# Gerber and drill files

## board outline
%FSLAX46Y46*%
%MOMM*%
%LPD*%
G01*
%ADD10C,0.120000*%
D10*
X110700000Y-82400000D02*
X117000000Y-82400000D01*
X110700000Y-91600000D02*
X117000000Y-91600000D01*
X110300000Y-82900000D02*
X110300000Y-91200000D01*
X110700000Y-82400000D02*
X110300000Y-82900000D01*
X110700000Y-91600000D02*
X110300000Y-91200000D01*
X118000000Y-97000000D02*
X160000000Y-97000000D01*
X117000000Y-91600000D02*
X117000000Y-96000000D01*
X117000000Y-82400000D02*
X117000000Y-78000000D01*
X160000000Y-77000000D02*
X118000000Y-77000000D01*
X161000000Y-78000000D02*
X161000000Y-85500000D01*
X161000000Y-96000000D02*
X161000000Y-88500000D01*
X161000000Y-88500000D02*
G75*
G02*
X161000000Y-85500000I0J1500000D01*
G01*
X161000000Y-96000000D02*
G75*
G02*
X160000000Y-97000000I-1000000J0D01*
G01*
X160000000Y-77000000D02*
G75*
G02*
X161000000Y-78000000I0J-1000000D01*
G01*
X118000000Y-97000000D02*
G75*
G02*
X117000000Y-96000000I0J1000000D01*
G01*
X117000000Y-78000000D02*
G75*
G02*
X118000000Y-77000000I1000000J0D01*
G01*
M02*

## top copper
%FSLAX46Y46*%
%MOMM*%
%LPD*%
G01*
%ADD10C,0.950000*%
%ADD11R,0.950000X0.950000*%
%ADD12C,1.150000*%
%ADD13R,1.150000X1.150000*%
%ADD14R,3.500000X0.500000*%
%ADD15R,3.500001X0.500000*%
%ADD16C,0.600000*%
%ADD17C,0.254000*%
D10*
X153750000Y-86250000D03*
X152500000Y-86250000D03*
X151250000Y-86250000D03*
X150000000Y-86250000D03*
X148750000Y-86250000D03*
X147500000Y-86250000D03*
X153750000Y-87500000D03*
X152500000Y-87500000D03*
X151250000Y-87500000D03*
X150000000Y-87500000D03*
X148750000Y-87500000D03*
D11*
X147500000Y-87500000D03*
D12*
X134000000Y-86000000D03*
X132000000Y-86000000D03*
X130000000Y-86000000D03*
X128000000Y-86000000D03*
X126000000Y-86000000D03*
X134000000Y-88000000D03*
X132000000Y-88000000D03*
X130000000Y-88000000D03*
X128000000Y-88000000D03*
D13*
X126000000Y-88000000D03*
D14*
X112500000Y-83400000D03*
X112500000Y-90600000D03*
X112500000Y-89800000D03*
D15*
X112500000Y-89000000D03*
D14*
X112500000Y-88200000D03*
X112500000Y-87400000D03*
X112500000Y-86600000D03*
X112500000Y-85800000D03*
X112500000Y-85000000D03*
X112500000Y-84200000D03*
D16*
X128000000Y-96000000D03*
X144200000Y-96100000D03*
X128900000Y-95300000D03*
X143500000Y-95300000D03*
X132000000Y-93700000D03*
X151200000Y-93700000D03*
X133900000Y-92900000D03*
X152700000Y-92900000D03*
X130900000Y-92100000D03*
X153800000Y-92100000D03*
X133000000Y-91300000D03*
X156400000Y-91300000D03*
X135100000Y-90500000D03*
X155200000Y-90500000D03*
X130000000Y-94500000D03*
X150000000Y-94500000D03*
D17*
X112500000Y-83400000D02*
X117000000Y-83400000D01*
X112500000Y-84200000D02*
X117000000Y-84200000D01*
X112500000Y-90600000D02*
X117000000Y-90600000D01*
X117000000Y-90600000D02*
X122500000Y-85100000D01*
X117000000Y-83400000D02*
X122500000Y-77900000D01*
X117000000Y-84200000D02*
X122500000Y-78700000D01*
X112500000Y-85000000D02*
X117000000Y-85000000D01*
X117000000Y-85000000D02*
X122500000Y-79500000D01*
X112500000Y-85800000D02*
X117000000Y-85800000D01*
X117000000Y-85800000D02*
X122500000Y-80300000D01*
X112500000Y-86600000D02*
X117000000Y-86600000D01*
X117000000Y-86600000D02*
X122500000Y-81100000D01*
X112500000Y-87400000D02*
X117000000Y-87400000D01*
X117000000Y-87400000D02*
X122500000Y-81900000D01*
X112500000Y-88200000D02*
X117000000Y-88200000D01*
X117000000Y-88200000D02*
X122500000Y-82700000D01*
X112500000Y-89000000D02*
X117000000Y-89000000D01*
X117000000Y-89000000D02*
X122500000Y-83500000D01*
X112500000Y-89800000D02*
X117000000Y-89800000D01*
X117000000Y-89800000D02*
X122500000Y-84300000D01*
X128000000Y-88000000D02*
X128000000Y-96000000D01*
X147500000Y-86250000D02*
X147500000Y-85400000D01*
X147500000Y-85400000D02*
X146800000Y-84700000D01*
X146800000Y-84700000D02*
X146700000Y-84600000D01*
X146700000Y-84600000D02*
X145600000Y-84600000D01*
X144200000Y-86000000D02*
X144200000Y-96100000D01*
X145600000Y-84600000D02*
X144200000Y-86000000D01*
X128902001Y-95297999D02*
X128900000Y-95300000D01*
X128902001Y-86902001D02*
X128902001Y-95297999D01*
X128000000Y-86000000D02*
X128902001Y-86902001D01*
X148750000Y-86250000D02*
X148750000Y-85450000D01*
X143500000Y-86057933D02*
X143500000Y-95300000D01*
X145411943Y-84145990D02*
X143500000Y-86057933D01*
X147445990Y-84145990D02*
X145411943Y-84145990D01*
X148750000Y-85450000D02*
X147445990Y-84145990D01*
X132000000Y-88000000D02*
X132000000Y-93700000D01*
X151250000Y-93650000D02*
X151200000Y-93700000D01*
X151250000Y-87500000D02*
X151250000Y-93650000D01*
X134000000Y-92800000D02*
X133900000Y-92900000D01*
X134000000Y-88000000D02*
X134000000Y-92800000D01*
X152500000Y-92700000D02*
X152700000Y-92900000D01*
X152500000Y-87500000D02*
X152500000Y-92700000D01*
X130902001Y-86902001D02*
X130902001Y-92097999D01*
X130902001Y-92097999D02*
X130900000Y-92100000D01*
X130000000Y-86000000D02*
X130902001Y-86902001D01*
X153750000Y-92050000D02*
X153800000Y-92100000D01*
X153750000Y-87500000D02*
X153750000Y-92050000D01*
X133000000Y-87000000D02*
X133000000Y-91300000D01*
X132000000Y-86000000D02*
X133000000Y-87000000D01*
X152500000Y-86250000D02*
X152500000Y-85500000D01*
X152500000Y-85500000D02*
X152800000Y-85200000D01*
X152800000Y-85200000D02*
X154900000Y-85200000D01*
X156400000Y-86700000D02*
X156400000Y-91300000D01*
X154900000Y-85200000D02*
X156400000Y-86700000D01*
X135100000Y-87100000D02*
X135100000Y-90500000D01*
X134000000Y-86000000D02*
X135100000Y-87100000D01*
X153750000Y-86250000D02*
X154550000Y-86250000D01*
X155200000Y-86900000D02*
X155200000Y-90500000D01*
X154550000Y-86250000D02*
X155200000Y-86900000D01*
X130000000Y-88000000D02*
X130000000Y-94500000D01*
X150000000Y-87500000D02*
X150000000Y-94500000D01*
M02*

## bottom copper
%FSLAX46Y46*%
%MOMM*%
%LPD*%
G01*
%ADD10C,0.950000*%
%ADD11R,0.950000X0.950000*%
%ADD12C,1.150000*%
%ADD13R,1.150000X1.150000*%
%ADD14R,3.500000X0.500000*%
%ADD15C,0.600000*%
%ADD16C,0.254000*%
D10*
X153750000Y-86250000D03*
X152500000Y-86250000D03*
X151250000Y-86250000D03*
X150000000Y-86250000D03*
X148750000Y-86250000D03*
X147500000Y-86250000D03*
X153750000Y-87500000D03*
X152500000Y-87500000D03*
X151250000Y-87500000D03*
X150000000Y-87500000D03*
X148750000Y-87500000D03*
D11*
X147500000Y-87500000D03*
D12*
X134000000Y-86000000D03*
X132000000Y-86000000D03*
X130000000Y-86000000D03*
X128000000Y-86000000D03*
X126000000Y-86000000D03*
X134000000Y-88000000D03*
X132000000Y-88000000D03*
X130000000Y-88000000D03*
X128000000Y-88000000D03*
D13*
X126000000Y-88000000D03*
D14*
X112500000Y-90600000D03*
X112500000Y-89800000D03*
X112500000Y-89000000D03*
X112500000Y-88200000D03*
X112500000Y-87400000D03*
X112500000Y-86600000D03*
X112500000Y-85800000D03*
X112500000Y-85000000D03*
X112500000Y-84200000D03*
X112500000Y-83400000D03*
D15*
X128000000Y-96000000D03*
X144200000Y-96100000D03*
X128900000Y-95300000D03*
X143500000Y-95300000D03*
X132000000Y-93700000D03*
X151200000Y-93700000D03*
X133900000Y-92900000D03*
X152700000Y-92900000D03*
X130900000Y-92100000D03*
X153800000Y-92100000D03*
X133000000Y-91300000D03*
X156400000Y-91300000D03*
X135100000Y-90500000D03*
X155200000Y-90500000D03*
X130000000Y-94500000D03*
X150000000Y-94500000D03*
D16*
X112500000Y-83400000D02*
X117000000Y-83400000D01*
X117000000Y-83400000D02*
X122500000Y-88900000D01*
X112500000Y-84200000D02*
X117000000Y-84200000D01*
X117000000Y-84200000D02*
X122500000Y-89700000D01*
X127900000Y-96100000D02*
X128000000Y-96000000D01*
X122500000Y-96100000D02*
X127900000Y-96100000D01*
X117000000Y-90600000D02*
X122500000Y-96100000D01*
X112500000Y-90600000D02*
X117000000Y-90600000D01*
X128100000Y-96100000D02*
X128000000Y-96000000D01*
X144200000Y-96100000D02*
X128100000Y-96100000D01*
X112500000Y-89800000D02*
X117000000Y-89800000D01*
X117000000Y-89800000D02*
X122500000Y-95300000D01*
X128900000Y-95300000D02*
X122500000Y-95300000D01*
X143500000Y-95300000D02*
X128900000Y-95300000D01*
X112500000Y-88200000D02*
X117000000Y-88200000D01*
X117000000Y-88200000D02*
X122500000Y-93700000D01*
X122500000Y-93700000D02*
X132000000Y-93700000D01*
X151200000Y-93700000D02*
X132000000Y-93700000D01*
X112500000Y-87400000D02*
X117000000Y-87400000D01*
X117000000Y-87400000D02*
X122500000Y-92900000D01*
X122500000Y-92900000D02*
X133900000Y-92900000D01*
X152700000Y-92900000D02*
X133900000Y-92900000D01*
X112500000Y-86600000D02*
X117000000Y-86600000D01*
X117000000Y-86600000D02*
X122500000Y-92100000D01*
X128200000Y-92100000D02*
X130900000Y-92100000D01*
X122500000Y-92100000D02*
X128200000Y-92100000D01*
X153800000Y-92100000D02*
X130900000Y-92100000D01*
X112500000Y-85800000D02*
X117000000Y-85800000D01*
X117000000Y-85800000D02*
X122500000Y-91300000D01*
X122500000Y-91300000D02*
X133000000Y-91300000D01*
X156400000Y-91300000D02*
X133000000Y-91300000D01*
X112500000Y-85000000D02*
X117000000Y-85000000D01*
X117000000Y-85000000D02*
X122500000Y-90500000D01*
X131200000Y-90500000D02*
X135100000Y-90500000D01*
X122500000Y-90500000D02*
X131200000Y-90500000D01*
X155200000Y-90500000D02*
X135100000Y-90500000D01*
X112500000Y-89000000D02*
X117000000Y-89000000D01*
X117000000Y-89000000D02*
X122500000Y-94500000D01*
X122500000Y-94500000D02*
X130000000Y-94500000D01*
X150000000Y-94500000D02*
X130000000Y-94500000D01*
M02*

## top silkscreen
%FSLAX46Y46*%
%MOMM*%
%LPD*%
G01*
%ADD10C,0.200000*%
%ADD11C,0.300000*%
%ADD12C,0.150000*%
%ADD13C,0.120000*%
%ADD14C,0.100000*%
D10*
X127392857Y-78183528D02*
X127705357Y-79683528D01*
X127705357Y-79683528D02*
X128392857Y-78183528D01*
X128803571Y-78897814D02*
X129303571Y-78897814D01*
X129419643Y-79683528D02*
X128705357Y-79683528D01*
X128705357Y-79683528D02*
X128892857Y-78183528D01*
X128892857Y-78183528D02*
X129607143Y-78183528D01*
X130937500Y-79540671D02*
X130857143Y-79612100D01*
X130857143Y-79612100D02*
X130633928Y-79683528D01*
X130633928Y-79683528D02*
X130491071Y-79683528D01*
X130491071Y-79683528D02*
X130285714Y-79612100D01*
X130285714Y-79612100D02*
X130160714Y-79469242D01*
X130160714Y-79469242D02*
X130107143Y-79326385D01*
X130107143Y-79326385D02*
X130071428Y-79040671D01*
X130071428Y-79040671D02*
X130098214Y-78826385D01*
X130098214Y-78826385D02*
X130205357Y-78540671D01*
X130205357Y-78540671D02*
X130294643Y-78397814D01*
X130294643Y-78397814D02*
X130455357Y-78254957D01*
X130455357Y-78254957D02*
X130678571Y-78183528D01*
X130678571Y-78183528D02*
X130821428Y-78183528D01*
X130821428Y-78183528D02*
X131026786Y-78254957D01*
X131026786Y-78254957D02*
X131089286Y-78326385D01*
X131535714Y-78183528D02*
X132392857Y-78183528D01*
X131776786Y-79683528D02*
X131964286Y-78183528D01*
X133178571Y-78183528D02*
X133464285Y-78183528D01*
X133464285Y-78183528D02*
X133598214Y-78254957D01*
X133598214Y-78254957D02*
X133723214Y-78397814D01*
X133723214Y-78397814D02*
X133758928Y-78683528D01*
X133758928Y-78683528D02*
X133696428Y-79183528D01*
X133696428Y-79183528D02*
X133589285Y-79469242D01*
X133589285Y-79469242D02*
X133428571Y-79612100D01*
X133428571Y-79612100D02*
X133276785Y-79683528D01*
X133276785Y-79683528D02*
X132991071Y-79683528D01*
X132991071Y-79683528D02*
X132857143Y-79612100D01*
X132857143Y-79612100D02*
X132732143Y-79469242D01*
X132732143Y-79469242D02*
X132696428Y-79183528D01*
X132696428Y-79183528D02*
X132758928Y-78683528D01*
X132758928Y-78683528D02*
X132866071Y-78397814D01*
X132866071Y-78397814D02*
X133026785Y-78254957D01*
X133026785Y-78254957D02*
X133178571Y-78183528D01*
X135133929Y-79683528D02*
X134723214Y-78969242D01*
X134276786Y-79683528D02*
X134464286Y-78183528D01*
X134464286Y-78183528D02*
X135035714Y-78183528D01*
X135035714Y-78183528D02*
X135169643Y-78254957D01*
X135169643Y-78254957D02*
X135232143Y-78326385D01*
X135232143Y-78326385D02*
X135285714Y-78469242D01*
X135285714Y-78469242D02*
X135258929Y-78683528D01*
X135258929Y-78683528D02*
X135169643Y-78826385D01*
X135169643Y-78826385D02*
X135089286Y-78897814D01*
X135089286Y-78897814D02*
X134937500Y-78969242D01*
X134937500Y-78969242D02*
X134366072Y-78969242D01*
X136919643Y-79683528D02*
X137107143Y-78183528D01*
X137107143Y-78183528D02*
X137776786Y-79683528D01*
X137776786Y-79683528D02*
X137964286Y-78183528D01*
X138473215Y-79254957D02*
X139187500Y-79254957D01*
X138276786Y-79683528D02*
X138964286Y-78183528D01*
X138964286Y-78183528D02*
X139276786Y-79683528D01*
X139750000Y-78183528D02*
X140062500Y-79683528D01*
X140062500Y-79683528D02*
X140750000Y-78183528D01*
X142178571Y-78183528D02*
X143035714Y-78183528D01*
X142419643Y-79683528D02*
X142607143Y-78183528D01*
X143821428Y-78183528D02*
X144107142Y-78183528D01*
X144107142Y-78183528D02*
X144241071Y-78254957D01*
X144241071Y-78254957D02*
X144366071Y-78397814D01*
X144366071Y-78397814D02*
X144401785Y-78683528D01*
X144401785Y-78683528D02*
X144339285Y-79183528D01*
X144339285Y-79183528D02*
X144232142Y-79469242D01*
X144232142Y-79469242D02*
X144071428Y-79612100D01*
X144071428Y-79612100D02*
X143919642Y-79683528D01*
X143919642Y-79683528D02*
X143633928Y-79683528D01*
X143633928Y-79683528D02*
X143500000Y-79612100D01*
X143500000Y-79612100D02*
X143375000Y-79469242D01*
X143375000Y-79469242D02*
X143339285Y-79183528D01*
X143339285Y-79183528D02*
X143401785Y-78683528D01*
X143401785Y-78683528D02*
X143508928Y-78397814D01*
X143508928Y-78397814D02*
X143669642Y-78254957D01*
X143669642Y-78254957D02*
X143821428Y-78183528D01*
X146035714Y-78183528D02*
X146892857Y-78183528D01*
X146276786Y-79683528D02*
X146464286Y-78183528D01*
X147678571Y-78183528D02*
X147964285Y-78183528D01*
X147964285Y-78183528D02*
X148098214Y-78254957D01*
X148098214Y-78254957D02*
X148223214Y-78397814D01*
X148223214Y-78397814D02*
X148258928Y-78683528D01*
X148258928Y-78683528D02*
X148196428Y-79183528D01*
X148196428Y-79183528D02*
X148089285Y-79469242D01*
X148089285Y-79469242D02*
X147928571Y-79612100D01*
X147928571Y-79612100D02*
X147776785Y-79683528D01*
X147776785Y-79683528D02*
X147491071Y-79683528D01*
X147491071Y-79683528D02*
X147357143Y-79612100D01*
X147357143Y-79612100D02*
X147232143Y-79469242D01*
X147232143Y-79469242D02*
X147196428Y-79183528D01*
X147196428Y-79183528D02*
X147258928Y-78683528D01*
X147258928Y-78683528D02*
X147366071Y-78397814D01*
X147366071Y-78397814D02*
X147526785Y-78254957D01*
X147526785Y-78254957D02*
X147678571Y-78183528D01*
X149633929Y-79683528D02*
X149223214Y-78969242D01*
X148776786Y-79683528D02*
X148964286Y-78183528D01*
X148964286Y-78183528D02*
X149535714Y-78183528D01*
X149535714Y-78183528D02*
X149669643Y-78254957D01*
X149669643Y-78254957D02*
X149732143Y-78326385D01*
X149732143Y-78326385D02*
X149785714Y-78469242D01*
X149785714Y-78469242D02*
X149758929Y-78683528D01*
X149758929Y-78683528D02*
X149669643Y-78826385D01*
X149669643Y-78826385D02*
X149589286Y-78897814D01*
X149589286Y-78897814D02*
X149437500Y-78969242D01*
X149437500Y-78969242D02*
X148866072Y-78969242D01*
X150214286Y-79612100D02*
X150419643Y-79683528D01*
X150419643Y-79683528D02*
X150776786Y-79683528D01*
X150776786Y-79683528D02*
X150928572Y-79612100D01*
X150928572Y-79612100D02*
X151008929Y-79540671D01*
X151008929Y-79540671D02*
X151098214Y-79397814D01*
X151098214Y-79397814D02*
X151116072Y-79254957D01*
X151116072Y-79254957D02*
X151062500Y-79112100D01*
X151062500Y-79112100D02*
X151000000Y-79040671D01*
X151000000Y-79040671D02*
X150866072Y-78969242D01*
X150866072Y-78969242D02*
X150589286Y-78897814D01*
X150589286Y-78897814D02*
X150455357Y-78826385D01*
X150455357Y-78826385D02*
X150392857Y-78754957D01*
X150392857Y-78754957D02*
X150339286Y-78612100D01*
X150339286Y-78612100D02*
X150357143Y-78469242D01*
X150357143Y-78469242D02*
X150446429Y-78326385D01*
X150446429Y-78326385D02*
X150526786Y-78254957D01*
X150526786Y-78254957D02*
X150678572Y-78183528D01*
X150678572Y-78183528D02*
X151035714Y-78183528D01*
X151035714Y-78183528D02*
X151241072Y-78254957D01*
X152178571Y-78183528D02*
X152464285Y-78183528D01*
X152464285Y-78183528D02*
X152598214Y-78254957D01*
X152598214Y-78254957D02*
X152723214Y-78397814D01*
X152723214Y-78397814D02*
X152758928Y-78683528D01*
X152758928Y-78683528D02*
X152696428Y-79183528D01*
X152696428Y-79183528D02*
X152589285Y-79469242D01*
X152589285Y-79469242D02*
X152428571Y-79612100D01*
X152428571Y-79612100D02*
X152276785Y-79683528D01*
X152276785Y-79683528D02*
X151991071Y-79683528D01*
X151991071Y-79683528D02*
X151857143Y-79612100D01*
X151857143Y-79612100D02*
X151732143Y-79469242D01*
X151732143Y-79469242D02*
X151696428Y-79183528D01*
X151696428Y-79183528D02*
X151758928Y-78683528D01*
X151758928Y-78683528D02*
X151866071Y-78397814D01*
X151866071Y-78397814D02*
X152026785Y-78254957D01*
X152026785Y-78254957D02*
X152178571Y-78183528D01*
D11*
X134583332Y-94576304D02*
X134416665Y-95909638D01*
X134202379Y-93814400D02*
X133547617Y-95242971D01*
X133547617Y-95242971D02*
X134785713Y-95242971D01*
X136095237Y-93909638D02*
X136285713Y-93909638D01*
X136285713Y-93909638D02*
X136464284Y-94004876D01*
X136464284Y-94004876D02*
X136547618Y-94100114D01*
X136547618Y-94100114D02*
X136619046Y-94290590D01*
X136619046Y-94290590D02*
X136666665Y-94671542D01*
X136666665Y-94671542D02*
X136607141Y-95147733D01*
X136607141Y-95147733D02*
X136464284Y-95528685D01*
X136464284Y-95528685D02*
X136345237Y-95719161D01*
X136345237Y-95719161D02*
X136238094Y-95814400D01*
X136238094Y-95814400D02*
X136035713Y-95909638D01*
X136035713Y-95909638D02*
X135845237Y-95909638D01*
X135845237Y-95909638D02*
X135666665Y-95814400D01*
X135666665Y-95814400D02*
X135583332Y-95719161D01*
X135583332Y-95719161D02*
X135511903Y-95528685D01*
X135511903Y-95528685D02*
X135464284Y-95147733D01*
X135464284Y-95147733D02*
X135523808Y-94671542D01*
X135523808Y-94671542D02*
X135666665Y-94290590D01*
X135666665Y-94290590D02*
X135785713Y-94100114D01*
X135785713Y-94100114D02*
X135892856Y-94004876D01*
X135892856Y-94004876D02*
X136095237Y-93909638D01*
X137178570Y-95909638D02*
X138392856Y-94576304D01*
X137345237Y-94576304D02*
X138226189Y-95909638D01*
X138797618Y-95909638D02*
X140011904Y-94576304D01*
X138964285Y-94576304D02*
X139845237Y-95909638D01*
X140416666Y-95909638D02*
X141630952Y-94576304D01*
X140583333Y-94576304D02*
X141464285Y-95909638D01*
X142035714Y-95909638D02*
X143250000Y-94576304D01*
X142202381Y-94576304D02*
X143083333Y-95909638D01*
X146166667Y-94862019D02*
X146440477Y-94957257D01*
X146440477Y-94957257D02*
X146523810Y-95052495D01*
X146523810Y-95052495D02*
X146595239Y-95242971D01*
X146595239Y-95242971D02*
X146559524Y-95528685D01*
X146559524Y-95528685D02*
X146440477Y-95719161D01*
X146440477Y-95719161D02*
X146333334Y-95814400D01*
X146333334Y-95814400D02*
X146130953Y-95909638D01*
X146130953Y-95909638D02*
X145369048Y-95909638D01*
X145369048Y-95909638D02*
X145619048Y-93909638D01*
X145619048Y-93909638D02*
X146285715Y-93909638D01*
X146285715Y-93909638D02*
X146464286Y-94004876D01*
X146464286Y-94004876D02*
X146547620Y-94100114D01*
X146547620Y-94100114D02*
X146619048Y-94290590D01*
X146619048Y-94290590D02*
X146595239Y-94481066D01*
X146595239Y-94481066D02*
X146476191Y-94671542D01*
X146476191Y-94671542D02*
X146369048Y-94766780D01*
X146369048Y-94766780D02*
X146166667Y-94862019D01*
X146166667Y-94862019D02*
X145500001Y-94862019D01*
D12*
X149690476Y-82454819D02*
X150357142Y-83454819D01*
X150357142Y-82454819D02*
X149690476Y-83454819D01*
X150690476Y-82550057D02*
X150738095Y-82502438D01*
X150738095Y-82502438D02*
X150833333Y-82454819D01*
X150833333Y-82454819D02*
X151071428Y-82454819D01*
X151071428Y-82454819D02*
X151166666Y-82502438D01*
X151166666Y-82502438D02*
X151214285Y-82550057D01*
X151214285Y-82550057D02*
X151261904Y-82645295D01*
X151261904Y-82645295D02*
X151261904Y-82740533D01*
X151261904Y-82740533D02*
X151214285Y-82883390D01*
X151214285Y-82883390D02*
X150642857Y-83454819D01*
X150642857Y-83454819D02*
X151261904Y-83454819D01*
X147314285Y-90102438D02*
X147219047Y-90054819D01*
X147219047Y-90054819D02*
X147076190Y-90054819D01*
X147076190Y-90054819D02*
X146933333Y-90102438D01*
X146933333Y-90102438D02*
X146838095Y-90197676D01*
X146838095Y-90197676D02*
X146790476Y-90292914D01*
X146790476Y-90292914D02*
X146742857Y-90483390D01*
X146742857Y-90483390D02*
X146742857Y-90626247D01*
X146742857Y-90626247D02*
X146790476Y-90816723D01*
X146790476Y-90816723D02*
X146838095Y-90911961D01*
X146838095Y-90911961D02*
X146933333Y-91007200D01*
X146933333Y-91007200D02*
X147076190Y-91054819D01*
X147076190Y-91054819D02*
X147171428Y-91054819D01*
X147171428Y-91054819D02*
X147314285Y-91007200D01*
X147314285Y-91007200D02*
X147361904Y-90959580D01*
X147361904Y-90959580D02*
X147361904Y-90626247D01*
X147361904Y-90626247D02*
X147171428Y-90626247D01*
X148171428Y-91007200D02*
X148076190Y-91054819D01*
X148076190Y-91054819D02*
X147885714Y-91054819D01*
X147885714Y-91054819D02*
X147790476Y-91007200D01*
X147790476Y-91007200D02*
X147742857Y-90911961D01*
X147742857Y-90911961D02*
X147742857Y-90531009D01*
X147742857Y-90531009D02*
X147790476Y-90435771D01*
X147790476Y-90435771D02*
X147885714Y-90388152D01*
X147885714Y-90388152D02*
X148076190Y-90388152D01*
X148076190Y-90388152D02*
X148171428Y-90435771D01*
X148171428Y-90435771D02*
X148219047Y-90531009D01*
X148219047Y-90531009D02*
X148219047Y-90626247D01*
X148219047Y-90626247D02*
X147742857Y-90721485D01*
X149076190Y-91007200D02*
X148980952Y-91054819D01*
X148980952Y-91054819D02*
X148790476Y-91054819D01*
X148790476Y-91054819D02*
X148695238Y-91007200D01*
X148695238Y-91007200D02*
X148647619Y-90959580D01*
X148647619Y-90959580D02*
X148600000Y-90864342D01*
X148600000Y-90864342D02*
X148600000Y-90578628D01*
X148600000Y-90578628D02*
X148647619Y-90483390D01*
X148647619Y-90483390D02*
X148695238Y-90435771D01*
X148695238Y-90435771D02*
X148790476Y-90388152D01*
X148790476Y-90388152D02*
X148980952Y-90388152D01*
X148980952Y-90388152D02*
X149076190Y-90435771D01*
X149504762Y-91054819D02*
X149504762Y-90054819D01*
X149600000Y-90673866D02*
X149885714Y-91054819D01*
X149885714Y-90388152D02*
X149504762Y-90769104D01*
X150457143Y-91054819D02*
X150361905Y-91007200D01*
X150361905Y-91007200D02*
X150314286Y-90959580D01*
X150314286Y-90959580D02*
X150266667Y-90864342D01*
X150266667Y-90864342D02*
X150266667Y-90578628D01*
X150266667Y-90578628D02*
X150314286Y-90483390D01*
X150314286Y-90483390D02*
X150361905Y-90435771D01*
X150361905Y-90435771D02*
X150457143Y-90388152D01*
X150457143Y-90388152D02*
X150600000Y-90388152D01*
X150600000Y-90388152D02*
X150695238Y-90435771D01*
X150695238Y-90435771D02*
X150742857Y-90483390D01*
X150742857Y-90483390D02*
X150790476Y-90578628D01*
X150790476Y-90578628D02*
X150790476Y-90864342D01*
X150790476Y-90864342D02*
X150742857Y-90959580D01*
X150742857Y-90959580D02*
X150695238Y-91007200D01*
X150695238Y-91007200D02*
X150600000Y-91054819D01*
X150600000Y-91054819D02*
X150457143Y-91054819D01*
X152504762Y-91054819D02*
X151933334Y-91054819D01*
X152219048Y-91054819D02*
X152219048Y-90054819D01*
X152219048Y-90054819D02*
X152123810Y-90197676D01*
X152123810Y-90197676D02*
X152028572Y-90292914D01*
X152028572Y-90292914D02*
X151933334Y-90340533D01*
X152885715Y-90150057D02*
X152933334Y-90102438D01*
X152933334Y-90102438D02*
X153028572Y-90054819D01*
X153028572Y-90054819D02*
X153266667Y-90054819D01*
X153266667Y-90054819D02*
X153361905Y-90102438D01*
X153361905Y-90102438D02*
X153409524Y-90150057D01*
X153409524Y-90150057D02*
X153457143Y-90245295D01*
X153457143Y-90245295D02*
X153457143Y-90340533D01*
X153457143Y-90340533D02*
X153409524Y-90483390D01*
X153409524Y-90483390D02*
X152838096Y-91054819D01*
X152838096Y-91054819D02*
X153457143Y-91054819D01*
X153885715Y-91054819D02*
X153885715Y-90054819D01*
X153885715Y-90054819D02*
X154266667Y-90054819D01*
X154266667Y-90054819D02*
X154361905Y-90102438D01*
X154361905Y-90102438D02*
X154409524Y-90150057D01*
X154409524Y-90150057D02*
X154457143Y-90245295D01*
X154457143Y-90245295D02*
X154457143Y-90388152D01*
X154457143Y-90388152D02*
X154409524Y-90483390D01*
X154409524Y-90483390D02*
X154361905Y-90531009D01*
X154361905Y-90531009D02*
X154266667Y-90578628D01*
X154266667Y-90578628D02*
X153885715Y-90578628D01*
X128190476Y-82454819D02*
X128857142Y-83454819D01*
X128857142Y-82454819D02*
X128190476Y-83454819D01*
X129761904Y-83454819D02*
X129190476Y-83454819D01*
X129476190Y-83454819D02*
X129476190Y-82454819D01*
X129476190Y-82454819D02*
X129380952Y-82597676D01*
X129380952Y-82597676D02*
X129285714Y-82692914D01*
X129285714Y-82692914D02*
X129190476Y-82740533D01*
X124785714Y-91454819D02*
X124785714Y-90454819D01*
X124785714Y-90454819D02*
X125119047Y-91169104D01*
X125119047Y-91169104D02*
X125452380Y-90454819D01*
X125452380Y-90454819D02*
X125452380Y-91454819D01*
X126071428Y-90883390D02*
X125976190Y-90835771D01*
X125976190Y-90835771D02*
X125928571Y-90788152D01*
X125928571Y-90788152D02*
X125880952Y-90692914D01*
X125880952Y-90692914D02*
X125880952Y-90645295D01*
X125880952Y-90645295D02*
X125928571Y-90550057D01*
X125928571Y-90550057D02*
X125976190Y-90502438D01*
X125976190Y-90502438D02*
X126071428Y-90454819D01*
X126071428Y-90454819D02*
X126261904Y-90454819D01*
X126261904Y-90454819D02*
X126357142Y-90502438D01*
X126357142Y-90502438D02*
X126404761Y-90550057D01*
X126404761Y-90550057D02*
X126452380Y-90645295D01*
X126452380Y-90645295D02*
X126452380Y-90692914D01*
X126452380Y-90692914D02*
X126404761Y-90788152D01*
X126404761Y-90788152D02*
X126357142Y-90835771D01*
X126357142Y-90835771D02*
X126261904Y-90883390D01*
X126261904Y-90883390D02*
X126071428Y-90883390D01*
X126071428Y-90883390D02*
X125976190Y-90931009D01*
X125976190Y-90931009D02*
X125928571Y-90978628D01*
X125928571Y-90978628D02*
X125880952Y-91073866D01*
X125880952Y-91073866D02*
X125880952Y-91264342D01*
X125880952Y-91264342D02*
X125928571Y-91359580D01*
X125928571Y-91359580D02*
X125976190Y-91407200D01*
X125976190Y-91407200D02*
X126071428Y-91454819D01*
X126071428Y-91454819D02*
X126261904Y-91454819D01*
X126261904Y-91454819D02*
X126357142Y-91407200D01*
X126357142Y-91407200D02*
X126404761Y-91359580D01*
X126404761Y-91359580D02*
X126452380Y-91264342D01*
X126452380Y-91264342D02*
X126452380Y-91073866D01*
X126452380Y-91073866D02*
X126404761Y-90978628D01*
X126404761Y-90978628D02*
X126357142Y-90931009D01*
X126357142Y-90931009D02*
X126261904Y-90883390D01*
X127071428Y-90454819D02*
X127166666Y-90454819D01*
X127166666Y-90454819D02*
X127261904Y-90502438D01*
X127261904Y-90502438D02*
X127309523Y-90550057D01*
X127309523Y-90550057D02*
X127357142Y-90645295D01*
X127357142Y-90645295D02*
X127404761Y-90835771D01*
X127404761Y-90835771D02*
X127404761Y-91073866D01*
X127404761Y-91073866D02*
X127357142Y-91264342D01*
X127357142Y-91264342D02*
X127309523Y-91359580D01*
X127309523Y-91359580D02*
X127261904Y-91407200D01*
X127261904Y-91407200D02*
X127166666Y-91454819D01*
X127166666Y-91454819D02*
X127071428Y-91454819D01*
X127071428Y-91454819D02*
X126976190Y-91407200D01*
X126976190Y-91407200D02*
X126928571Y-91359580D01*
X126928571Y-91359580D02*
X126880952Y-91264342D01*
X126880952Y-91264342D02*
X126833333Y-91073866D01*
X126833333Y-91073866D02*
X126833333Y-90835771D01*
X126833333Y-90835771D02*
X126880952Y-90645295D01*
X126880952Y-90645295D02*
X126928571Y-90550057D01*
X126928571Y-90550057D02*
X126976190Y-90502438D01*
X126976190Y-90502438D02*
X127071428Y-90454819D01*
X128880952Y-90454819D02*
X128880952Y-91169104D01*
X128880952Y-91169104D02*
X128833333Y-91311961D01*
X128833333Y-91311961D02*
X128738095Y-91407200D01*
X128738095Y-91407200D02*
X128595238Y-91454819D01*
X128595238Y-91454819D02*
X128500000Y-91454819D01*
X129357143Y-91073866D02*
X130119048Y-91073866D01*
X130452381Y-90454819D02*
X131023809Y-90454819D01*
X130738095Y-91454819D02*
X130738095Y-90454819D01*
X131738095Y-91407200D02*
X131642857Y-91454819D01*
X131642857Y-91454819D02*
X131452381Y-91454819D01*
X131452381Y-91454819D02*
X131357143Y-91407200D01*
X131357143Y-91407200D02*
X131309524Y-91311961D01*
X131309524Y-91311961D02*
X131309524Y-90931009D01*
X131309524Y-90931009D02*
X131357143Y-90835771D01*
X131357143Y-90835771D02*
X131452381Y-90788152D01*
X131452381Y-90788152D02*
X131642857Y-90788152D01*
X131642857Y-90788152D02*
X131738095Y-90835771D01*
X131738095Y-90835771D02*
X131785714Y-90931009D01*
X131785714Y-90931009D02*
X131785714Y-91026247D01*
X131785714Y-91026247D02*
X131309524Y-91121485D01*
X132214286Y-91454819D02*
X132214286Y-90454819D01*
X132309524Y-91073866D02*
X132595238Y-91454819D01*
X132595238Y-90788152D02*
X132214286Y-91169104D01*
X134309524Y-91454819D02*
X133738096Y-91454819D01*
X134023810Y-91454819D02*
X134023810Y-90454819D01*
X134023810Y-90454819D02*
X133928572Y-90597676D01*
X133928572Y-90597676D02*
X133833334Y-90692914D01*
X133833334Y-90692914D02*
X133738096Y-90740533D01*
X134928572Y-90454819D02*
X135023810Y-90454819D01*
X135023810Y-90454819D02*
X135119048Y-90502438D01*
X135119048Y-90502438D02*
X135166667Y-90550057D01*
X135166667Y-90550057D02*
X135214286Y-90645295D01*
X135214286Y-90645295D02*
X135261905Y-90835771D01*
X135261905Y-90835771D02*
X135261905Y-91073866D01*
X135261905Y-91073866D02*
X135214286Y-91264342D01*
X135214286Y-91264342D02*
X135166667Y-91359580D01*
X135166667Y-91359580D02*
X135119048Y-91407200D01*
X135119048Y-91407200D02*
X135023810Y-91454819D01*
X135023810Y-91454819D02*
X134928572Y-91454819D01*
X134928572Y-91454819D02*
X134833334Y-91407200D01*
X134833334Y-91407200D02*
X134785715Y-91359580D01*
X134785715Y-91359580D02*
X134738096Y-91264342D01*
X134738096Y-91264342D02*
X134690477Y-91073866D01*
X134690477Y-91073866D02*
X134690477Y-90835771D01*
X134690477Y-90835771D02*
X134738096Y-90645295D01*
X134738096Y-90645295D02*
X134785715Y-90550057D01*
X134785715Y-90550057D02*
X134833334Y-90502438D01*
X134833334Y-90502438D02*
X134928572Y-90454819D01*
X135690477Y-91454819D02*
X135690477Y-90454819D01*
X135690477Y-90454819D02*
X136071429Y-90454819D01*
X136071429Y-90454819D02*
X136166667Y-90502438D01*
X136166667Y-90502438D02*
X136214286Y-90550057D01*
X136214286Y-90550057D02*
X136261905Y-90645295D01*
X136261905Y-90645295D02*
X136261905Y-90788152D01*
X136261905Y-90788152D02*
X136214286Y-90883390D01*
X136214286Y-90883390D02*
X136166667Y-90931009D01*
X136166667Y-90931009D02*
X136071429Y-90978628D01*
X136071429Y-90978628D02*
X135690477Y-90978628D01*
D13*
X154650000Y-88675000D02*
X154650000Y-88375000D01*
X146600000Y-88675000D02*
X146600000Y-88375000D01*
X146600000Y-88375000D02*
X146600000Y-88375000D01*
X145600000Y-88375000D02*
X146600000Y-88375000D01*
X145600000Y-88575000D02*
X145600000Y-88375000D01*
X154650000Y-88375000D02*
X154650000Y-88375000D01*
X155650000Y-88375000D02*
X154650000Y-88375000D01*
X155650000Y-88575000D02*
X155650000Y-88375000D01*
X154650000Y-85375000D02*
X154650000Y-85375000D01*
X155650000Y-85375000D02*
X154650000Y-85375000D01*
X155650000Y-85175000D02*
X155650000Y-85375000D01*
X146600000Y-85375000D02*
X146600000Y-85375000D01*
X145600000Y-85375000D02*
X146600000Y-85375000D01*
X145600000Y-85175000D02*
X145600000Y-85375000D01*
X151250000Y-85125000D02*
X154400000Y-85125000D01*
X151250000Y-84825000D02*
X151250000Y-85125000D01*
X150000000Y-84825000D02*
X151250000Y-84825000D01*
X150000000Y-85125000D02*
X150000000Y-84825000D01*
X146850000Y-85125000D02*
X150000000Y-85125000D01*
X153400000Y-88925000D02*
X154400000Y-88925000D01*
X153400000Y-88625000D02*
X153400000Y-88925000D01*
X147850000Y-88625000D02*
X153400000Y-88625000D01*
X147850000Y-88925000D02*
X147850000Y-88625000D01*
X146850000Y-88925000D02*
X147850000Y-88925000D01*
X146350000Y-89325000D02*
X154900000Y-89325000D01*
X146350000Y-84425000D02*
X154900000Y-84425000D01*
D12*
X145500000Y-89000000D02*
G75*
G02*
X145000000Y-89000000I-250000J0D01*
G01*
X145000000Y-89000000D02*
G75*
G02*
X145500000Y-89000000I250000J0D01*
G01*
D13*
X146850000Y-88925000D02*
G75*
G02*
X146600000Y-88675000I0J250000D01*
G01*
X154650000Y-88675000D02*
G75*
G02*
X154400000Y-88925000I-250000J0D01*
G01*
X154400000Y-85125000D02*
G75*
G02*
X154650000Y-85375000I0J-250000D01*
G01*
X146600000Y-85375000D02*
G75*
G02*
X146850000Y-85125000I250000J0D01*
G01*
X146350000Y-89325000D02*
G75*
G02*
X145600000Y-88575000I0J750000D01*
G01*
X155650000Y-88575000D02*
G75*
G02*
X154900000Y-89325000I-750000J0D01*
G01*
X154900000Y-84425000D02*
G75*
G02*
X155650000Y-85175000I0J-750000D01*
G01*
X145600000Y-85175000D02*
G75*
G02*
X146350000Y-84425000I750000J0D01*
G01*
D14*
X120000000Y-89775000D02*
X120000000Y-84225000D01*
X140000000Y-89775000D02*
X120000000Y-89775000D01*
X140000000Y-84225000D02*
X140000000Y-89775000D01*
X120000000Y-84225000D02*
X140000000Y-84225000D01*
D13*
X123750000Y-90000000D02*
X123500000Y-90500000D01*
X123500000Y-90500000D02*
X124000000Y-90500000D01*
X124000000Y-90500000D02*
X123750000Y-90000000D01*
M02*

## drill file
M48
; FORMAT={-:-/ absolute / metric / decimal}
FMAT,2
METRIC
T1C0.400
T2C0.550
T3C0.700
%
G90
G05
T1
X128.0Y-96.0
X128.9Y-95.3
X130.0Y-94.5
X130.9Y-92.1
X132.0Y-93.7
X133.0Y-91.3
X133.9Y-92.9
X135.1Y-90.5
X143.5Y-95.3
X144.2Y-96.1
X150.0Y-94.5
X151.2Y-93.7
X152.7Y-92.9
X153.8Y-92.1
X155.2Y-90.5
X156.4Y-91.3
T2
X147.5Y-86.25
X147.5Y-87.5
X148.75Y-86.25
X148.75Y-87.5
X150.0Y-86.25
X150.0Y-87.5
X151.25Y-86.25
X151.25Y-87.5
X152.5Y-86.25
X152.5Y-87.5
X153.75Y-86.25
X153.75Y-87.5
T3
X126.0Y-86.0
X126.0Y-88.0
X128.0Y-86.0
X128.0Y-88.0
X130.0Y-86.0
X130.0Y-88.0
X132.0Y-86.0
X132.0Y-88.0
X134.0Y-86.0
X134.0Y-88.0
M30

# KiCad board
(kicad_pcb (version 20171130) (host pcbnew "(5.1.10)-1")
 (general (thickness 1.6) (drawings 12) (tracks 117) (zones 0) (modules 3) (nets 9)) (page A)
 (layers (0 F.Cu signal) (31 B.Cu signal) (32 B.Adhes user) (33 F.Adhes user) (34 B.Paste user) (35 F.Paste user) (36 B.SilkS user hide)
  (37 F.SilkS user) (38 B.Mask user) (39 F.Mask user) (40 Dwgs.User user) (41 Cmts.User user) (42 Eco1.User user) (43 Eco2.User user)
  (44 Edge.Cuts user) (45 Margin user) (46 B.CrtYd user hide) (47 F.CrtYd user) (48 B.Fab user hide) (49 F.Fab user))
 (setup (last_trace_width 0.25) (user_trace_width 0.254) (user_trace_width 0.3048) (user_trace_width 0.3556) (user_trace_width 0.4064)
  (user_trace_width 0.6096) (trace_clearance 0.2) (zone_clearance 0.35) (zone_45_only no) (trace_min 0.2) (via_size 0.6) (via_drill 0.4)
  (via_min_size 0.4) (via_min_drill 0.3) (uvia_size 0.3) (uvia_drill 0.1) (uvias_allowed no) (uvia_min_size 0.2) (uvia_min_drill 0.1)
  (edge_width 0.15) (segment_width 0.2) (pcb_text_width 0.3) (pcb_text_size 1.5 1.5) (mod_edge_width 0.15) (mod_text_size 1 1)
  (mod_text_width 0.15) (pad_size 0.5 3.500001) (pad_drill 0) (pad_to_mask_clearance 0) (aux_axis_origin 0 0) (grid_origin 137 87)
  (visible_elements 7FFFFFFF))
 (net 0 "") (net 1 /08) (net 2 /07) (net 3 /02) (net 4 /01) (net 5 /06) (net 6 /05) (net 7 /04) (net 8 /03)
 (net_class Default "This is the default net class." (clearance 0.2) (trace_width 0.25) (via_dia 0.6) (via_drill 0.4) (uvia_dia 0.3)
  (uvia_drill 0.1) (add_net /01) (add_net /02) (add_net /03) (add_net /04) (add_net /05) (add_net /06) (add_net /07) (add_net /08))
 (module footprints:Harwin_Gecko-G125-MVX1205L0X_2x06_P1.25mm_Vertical (layer F.Cu) (at 147.5 87.5)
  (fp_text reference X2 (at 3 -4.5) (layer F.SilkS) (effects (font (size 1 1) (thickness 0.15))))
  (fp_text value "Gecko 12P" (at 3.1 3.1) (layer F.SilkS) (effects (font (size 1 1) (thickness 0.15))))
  (fp_line (start 7.15 1.175) (end 7.15 0.875) (layer F.SilkS) (width 0.12))
  (fp_line (start -0.9 1.175) (end -0.9 0.875) (layer F.SilkS) (width 0.12))
  (fp_line (start -0.9 0.875) (end -0.9 0.875) (layer F.SilkS) (width 0.12))
  (fp_line (start -1.9 0.875) (end -0.9 0.875) (layer F.SilkS) (width 0.12))
  (fp_line (start -1.9 1.075) (end -1.9 0.875) (layer F.SilkS) (width 0.12))
  (fp_line (start 7.15 0.875) (end 7.15 0.875) (layer F.SilkS) (width 0.12))
  (fp_line (start 8.15 0.875) (end 7.15 0.875) (layer F.SilkS) (width 0.12))
  (fp_line (start 8.15 1.075) (end 8.15 0.875) (layer F.SilkS) (width 0.12))
  (fp_line (start 7.15 -2.125) (end 7.15 -2.125) (layer F.SilkS) (width 0.12))
  (fp_line (start 8.15 -2.125) (end 7.15 -2.125) (layer F.SilkS) (width 0.12))
  (fp_line (start 8.15 -2.325) (end 8.15 -2.125) (layer F.SilkS) (width 0.12))
  (fp_line (start -0.9 -2.125) (end -0.9 -2.125) (layer F.SilkS) (width 0.12))
  (fp_line (start -1.9 -2.125) (end -0.9 -2.125) (layer F.SilkS) (width 0.12))
  (fp_line (start -1.9 -2.325) (end -1.9 -2.125) (layer F.SilkS) (width 0.12))
  (fp_line (start 3.75 -2.375) (end 6.9 -2.375) (layer F.SilkS) (width 0.12))
  (fp_line (start 3.75 -2.675) (end 3.75 -2.375) (layer F.SilkS) (width 0.12))
  (fp_line (start 2.5 -2.675) (end 3.75 -2.675) (layer F.SilkS) (width 0.12))
  (fp_line (start 2.5 -2.375) (end 2.5 -2.675) (layer F.SilkS) (width 0.12))
  (fp_line (start -0.65 -2.375) (end 2.5 -2.375) (layer F.SilkS) (width 0.12))
  (fp_line (start 5.9 1.425) (end 6.9 1.425) (layer F.SilkS) (width 0.12))
  (fp_line (start 5.9 1.125) (end 5.9 1.425) (layer F.SilkS) (width 0.12))
  (fp_line (start 0.35 1.125) (end 5.9 1.125) (layer F.SilkS) (width 0.12))
  (fp_line (start 0.35 1.425) (end 0.35 1.125) (layer F.SilkS) (width 0.12))
  (fp_line (start -0.65 1.425) (end 0.35 1.425) (layer F.SilkS) (width 0.12))
  (fp_line (start -1.15 1.825) (end 7.4 1.825) (layer F.SilkS) (width 0.12))
  (fp_line (start -1.15 -3.075) (end 7.4 -3.075) (layer F.SilkS) (width 0.12))
  (fp_circle (center -2.25 1.5) (end -2 1.5) (layer F.SilkS) (width 0.15))
  (fp_arc (start -0.65 1.175) (end -0.65 1.425) (angle 90) (layer F.SilkS) (width 0.12))
  (fp_arc (start 6.9 1.175) (end 7.15 1.175) (angle 90) (layer F.SilkS) (width 0.12))
  (fp_arc (start 6.9 -2.125) (end 6.9 -2.375) (angle 90) (layer F.SilkS) (width 0.12))
  (fp_arc (start -0.65 -2.125) (end -0.9 -2.125) (angle 90) (layer F.SilkS) (width 0.12))
  (fp_arc (start -1.15 1.075) (end -1.15 1.825) (angle 90) (layer F.SilkS) (width 0.12))
  (fp_arc (start 7.4 1.075) (end 8.15 1.075) (angle 90) (layer F.SilkS) (width 0.12))
  (fp_arc (start 7.4 -2.325) (end 7.4 -3.075) (angle 90) (layer F.SilkS) (width 0.12))
  (fp_arc (start -1.15 -2.325) (end -1.9 -2.325) (angle 90) (layer F.SilkS) (width 0.12))
  (pad 12 thru_hole circle (at 6.25 -1.25) (size 0.95 0.95) (drill 0.55) (layers *.Cu *.Mask) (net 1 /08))
  (pad 11 thru_hole circle (at 5 -1.25) (size 0.95 0.95) (drill 0.55) (layers *.Cu *.Mask) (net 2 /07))
  (pad 10 thru_hole circle (at 3.75 -1.25) (size 0.95 0.95) (drill 0.55) (layers *.Cu *.Mask))
  (pad 9 thru_hole circle (at 2.5 -1.25) (size 0.95 0.95) (drill 0.55) (layers *.Cu *.Mask))
  (pad 8 thru_hole circle (at 1.25 -1.25) (size 0.95 0.95) (drill 0.55) (layers *.Cu *.Mask) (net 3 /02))
  (pad 7 thru_hole circle (at 0 -1.25) (size 0.95 0.95) (drill 0.55) (layers *.Cu *.Mask) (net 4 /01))
  (pad 6 thru_hole circle (at 6.25 0) (size 0.95 0.95) (drill 0.55) (layers *.Cu *.Mask) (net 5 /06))
  (pad 5 thru_hole circle (at 5 0) (size 0.95 0.95) (drill 0.55) (layers *.Cu *.Mask) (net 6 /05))
  (pad 4 thru_hole circle (at 3.75 0) (size 0.95 0.95) (drill 0.55) (layers *.Cu *.Mask) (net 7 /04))
  (pad 3 thru_hole circle (at 2.5 0) (size 0.95 0.95) (drill 0.55) (layers *.Cu *.Mask) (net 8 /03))
  (pad 2 thru_hole circle (at 1.25 0) (size 0.95 0.95) (drill 0.55) (layers *.Cu *.Mask))
  (pad 1 thru_hole rect (at 0 0) (size 0.95 0.95) (drill 0.55) (layers *.Cu *.Mask)))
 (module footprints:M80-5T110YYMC (layer F.Cu) (at 126 88)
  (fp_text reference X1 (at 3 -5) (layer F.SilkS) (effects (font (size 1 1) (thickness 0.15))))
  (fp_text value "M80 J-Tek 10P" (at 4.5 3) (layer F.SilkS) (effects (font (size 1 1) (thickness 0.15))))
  (fp_line (start -6 1.775) (end -6 -3.775) (layer F.SilkS) (width 0.1))
  (fp_line (start 14 1.775) (end -6 1.775) (layer F.SilkS) (width 0.1))
  (fp_line (start 14 -3.775) (end 14 1.775) (layer F.SilkS) (width 0.1))
  (fp_line (start -6 -3.775) (end 14 -3.775) (layer F.SilkS) (width 0.1))
  (fp_line (start -2.25 2) (end -2.5 2.5) (layer F.SilkS) (width 0.12))
  (fp_line (start -2.5 2.5) (end -2 2.5) (layer F.SilkS) (width 0.12))
  (fp_line (start -2 2.5) (end -2.25 2) (layer F.SilkS) (width 0.12))
  (pad 10 thru_hole circle (at 8 -2) (size 1.15 1.15) (drill 0.7) (layers *.Cu *.Mask) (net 1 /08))
  (pad 9 thru_hole circle (at 6 -2) (size 1.15 1.15) (drill 0.7) (layers *.Cu *.Mask) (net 2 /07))
  (pad 8 thru_hole circle (at 4 -2) (size 1.15 1.15) (drill 0.7) (layers *.Cu *.Mask) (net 5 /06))
  (pad 7 thru_hole circle (at 2 -2) (size 1.15 1.15) (drill 0.7) (layers *.Cu *.Mask) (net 3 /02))
  (pad 6 thru_hole circle (at 0 -2) (size 1.15 1.15) (drill 0.7) (layers *.Cu *.Mask))
  (pad 5 thru_hole circle (at 8 0) (size 1.15 1.15) (drill 0.7) (layers *.Cu *.Mask) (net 6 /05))
  (pad 4 thru_hole circle (at 6 0) (size 1.15 1.15) (drill 0.7) (layers *.Cu *.Mask) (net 7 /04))
  (pad 3 thru_hole circle (at 4 0) (size 1.15 1.15) (drill 0.7) (layers *.Cu *.Mask) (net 8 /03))
  (pad 2 thru_hole circle (at 2 0) (size 1.15 1.15) (drill 0.7) (layers *.Cu *.Mask) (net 4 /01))
  (pad 1 thru_hole rect (at 0 0) (size 1.15 1.15) (drill 0.7) (layers *.Cu *.Mask)))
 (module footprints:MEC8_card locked (layer F.Cu) (at 112.5 87 90)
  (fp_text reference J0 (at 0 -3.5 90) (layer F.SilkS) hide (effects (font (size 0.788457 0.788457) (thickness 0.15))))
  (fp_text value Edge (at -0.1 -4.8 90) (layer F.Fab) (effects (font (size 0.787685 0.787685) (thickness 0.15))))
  (fp_line (start 4.6 -1.8) (end 4.6 4.5) (layer Edge.Cuts) (width 0.12))
  (fp_line (start -4.6 -1.8) (end -4.6 4.5) (layer Edge.Cuts) (width 0.12))
  (fp_line (start 4.1 -2.2) (end -4.2 -2.2) (layer Edge.Cuts) (width 0.12))
  (fp_line (start 4.6 -1.8) (end 4.1 -2.2) (layer Edge.Cuts) (width 0.12))
  (fp_line (start -4.6 -1.8) (end -4.2 -2.2) (layer Edge.Cuts) (width 0.12))
  (fp_line (start -10 5.5) (end -10 47.5) (layer Edge.Cuts) (width 0.12))
  (fp_line (start -4.6 4.5) (end -9 4.5) (layer Edge.Cuts) (width 0.12))
  (fp_line (start 4.6 4.5) (end 9 4.5) (layer Edge.Cuts) (width 0.12))
  (fp_line (start 10 47.5) (end 10 5.5) (layer Edge.Cuts) (width 0.12))
  (fp_line (start 9 48.5) (end 1.5 48.5) (layer Edge.Cuts) (width 0.12))
  (fp_line (start -9 48.5) (end -1.5 48.5) (layer Edge.Cuts) (width 0.12))
  (fp_arc (start 0 48.5) (end 1.5 48.5) (angle -180) (layer Edge.Cuts) (width 0.12))
  (fp_arc (start -9 47.5) (end -10 47.5) (angle -90) (layer Edge.Cuts) (width 0.12))
  (fp_arc (start 9 47.5) (end 9 48.5) (angle -90) (layer Edge.Cuts) (width 0.12))
  (fp_arc (start -9 5.5) (end -9 4.5) (angle -90) (layer Edge.Cuts) (width 0.12))
  (fp_arc (start 9 5.5) (end 10 5.5) (angle -90) (layer Edge.Cuts) (width 0.12))
  (pad 20 smd rect (at 3.6 0 90) (size 0.5 3.5) (layers F.Cu F.Paste F.Mask))
  (pad 11 smd rect (at -3.6 0 90) (size 0.5 3.5) (layers F.Cu F.Paste F.Mask))
  (pad 12 smd rect (at -2.8 0 90) (size 0.5 3.5) (layers F.Cu F.Paste F.Mask))
  (pad 13 smd rect (at -2 0 90) (size 0.5 3.500001) (layers F.Cu F.Paste F.Mask))
  (pad 14 smd rect (at -1.2 0 90) (size 0.5 3.5) (layers F.Cu F.Paste F.Mask))
  (pad 15 smd rect (at -0.4 0 90) (size 0.5 3.5) (layers F.Cu F.Paste F.Mask))
  (pad 16 smd rect (at 0.4 0 90) (size 0.5 3.5) (layers F.Cu F.Paste F.Mask))
  (pad 17 smd rect (at 1.2 0 90) (size 0.5 3.5) (layers F.Cu F.Paste F.Mask))
  (pad 18 smd rect (at 2 0 90) (size 0.5 3.5) (layers F.Cu F.Paste F.Mask))
  (pad 19 smd rect (at 2.8 0 90) (size 0.5 3.5) (layers F.Cu F.Paste F.Mask))
  (pad 1 smd rect (at -3.6 0 90) (size 0.5 3.5) (layers B.Cu B.Paste B.Mask) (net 4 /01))
  (pad 2 smd rect (at -2.8 0 90) (size 0.5 3.5) (layers B.Cu B.Paste B.Mask) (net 3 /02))
  (pad 3 smd rect (at -2 0 90) (size 0.5 3.5) (layers B.Cu B.Paste B.Mask) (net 8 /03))
  (pad 4 smd rect (at -1.2 0 90) (size 0.5 3.5) (layers B.Cu B.Paste B.Mask) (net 7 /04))
  (pad 5 smd rect (at -0.4 0 90) (size 0.5 3.5) (layers B.Cu B.Paste B.Mask) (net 6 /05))
  (pad 6 smd rect (at 0.4 0 90) (size 0.5 3.5) (layers B.Cu B.Paste B.Mask) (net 5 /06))
  (pad 7 smd rect (at 1.2 0 90) (size 0.5 3.5) (layers B.Cu B.Paste B.Mask) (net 2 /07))
  (pad 8 smd rect (at 2 0 90) (size 0.5 3.5) (layers B.Cu B.Paste B.Mask) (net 1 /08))
  (pad 9 smd rect (at 2.8 0 90) (size 0.5 3.5) (layers B.Cu B.Paste B.Mask))
  (pad 10 smd rect (at 3.6 0 90) (size 0.5 3.5) (layers B.Cu B.Paste B.Mask)))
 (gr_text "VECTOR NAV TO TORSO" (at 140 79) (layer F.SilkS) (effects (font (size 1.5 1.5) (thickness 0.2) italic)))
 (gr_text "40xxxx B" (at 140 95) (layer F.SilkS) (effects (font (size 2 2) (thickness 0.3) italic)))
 (segment (start 112.5 83.4) (end 117 83.4) (width 0.254) (layer F.Cu) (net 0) (status 10))
 (segment (start 112.5 84.2) (end 117 84.2) (width 0.254) (layer F.Cu) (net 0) (status 10))
 (segment (start 112.5 90.6) (end 117 90.6) (width 0.254) (layer F.Cu) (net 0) (status 10))
 (segment (start 117 90.6) (end 122.5 85.1) (width 0.254) (layer F.Cu) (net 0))
 (segment (start 117 83.4) (end 122.5 77.9) (width 0.254) (layer F.Cu) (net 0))
 (segment (start 117 84.2) (end 122.5 78.7) (width 0.254) (layer F.Cu) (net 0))
 (segment (start 112.5 83.4) (end 117 83.4) (width 0.254) (layer B.Cu) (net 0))
 (segment (start 117 83.4) (end 122.5 88.9) (width 0.254) (layer B.Cu) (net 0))
 (segment (start 112.5 85) (end 117 85) (width 0.254) (layer F.Cu) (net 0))
 (segment (start 117 85) (end 122.5 79.5) (width 0.254) (layer F.Cu) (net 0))
 (segment (start 112.5 85.8) (end 117 85.8) (width 0.254) (layer F.Cu) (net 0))
 (segment (start 117 85.8) (end 122.5 80.3) (width 0.254) (layer F.Cu) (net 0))
 (segment (start 112.5 86.6) (end 117 86.6) (width 0.254) (layer F.Cu) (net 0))
 (segment (start 117 86.6) (end 122.5 81.1) (width 0.254) (layer F.Cu) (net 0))
 (segment (start 112.5 87.4) (end 117 87.4) (width 0.254) (layer F.Cu) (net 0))
 (segment (start 117 87.4) (end 122.5 81.9) (width 0.254) (layer F.Cu) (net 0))
 (segment (start 112.5 88.2) (end 117 88.2) (width 0.254) (layer F.Cu) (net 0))
 (segment (start 117 88.2) (end 122.5 82.7) (width 0.254) (layer F.Cu) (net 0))
 (segment (start 112.5 89) (end 117 89) (width 0.254) (layer F.Cu) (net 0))
 (segment (start 117 89) (end 122.5 83.5) (width 0.254) (layer F.Cu) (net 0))
 (segment (start 112.5 89.8) (end 117 89.8) (width 0.254) (layer F.Cu) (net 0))
 (segment (start 117 89.8) (end 122.5 84.3) (width 0.254) (layer F.Cu) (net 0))
 (segment (start 112.5 84.2) (end 117 84.2) (width 0.254) (layer B.Cu) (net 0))
 (segment (start 117 84.2) (end 122.5 89.7) (width 0.254) (layer B.Cu) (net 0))
 (via (at 128 96) (size 0.6) (drill 0.4) (layers F.Cu B.Cu) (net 4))
 (segment (start 128 88) (end 128 96) (width 0.254) (layer F.Cu) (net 4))
 (segment (start 127.9 96.1) (end 128 96) (width 0.254) (layer B.Cu) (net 4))
 (segment (start 122.5 96.1) (end 127.9 96.1) (width 0.254) (layer B.Cu) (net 4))
 (segment (start 117 90.6) (end 122.5 96.1) (width 0.254) (layer B.Cu) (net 4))
 (segment (start 112.5 90.6) (end 117 90.6) (width 0.254) (layer B.Cu) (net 4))
 (segment (start 147.5 86.25) (end 147.5 85.4) (width 0.254) (layer F.Cu) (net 4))
 (segment (start 147.5 85.4) (end 146.8 84.7) (width 0.254) (layer F.Cu) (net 4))
 (segment (start 146.8 84.7) (end 146.7 84.6) (width 0.254) (layer F.Cu) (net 4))
 (segment (start 146.7 84.6) (end 145.6 84.6) (width 0.254) (layer F.Cu) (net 4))
 (via (at 144.2 96.1) (size 0.6) (drill 0.4) (layers F.Cu B.Cu) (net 4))
 (segment (start 144.2 86) (end 144.2 96.1) (width 0.254) (layer F.Cu) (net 4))
 (segment (start 145.6 84.6) (end 144.2 86) (width 0.254) (layer F.Cu) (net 4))
 (segment (start 128.1 96.1) (end 128 96) (width 0.254) (layer B.Cu) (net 4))
 (segment (start 144.2 96.1) (end 128.1 96.1) (width 0.254) (layer B.Cu) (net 4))
 (segment (start 112.5 89.8) (end 117 89.8) (width 0.254) (layer B.Cu) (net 3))
 (segment (start 117 89.8) (end 122.5 95.3) (width 0.254) (layer B.Cu) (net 3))
 (via (at 128.9 95.3) (size 0.6) (drill 0.4) (layers F.Cu B.Cu) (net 3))
 (segment (start 128.902001 95.297999) (end 128.9 95.3) (width 0.254) (layer F.Cu) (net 3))
 (segment (start 128.902001 86.902001) (end 128.902001 95.297999) (width 0.254) (layer F.Cu) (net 3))
 (segment (start 128 86) (end 128.902001 86.902001) (width 0.254) (layer F.Cu) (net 3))
 (segment (start 128.9 95.3) (end 122.5 95.3) (width 0.254) (layer B.Cu) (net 3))
 (segment (start 148.75 86.25) (end 148.75 85.45) (width 0.254) (layer F.Cu) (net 3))
 (via (at 143.5 95.3) (size 0.6) (drill 0.4) (layers F.Cu B.Cu) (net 3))
 (segment (start 143.5 86.057933) (end 143.5 95.3) (width 0.254) (layer F.Cu) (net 3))
 (segment (start 145.411943 84.14599) (end 143.5 86.057933) (width 0.254) (layer F.Cu) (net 3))
 (segment (start 147.44599 84.14599) (end 145.411943 84.14599) (width 0.254) (layer F.Cu) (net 3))
 (segment (start 148.75 85.45) (end 147.44599 84.14599) (width 0.254) (layer F.Cu) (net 3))
 (segment (start 143.5 95.3) (end 128.9 95.3) (width 0.254) (layer B.Cu) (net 3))
 (segment (start 112.5 88.2) (end 117 88.2) (width 0.254) (layer B.Cu) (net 7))
 (segment (start 117 88.2) (end 122.5 93.7) (width 0.254) (layer B.Cu) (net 7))
 (via (at 132 93.7) (size 0.6) (drill 0.4) (layers F.Cu B.Cu) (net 7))
 (segment (start 132 88) (end 132 93.7) (width 0.254) (layer F.Cu) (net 7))
 (segment (start 122.5 93.7) (end 132 93.7) (width 0.254) (layer B.Cu) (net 7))
 (via (at 151.2 93.7) (size 0.6) (drill 0.4) (layers F.Cu B.Cu) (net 7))
 (segment (start 151.25 93.65) (end 151.2 93.7) (width 0.254) (layer F.Cu) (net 7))
 (segment (start 151.25 87.5) (end 151.25 93.65) (width 0.254) (layer F.Cu) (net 7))
 (segment (start 151.2 93.7) (end 132 93.7) (width 0.254) (layer B.Cu) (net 7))
 (segment (start 112.5 87.4) (end 117 87.4) (width 0.254) (layer B.Cu) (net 6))
 (segment (start 117 87.4) (end 122.5 92.9) (width 0.254) (layer B.Cu) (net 6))
 (via (at 133.9 92.9) (size 0.6) (drill 0.4) (layers F.Cu B.Cu) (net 6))
 (segment (start 134 92.8) (end 133.9 92.9) (width 0.254) (layer F.Cu) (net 6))
 (segment (start 134 88) (end 134 92.8) (width 0.254) (layer F.Cu) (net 6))
 (segment (start 122.5 92.9) (end 133.9 92.9) (width 0.254) (layer B.Cu) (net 6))
 (via (at 152.7 92.9) (size 0.6) (drill 0.4) (layers F.Cu B.Cu) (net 6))
 (segment (start 152.5 92.7) (end 152.7 92.9) (width 0.254) (layer F.Cu) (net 6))
 (segment (start 152.5 87.5) (end 152.5 92.7) (width 0.254) (layer F.Cu) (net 6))
 (segment (start 152.7 92.9) (end 133.9 92.9) (width 0.254) (layer B.Cu) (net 6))
 (segment (start 112.5 86.6) (end 117 86.6) (width 0.254) (layer B.Cu) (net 5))
 (segment (start 117 86.6) (end 122.5 92.1) (width 0.254) (layer B.Cu) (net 5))
 (via (at 130.9 92.1) (size 0.6) (drill 0.4) (layers F.Cu B.Cu) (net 5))
 (segment (start 130.902001 86.902001) (end 130.902001 92.097999) (width 0.254) (layer F.Cu) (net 5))
 (segment (start 130.902001 92.097999) (end 130.9 92.1) (width 0.254) (layer F.Cu) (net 5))
 (segment (start 130 86) (end 130.902001 86.902001) (width 0.254) (layer F.Cu) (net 5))
 (segment (start 128.2 92.1) (end 130.9 92.1) (width 0.254) (layer B.Cu) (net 5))
 (segment (start 122.5 92.1) (end 128.2 92.1) (width 0.254) (layer B.Cu) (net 5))
 (via (at 153.8 92.1) (size 0.6) (drill 0.4) (layers F.Cu B.Cu) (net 5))
 (segment (start 153.75 92.05) (end 153.8 92.1) (width 0.254) (layer F.Cu) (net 5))
 (segment (start 153.75 87.5) (end 153.75 92.05) (width 0.254) (layer F.Cu) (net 5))
 (segment (start 153.8 92.1) (end 130.9 92.1) (width 0.254) (layer B.Cu) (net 5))
 (segment (start 112.5 85.8) (end 117 85.8) (width 0.254) (layer B.Cu) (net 2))
 (segment (start 117 85.8) (end 122.5 91.3) (width 0.254) (layer B.Cu) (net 2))
 (via (at 133 91.3) (size 0.6) (drill 0.4) (layers F.Cu B.Cu) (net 2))
 (segment (start 133 87) (end 133 91.3) (width 0.254) (layer F.Cu) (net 2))
 (segment (start 132 86) (end 133 87) (width 0.254) (layer F.Cu) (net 2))
 (segment (start 122.5 91.3) (end 133 91.3) (width 0.254) (layer B.Cu) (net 2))
 (segment (start 152.5 86.25) (end 152.5 85.5) (width 0.254) (layer F.Cu) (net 2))
 (segment (start 152.5 85.5) (end 152.8 85.2) (width 0.254) (layer F.Cu) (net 2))
 (segment (start 152.8 85.2) (end 154.9 85.2) (width 0.254) (layer F.Cu) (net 2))
 (via (at 156.4 91.3) (size 0.6) (drill 0.4) (layers F.Cu B.Cu) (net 2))
 (segment (start 156.4 86.7) (end 156.4 91.3) (width 0.254) (layer F.Cu) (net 2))
 (segment (start 154.9 85.2) (end 156.4 86.7) (width 0.254) (layer F.Cu) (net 2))
 (segment (start 156.4 91.3) (end 133 91.3) (width 0.254) (layer B.Cu) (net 2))
 (segment (start 112.5 85) (end 117 85) (width 0.254) (layer B.Cu) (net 1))
 (segment (start 117 85) (end 122.5 90.5) (width 0.254) (layer B.Cu) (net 1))
 (via (at 135.1 90.5) (size 0.6) (drill 0.4) (layers F.Cu B.Cu) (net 1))
 (segment (start 135.1 87.1) (end 135.1 90.5) (width 0.254) (layer F.Cu) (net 1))
 (segment (start 134 86) (end 135.1 87.1) (width 0.254) (layer F.Cu) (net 1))
 (segment (start 131.2 90.5) (end 135.1 90.5) (width 0.254) (layer B.Cu) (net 1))
 (segment (start 122.5 90.5) (end 131.2 90.5) (width 0.254) (layer B.Cu) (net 1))
 (segment (start 153.75 86.25) (end 154.55 86.25) (width 0.254) (layer F.Cu) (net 1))
 (via (at 155.2 90.5) (size 0.6) (drill 0.4) (layers F.Cu B.Cu) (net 1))
 (segment (start 155.2 86.9) (end 155.2 90.5) (width 0.254) (layer F.Cu) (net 1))
 (segment (start 154.55 86.25) (end 155.2 86.9) (width 0.254) (layer F.Cu) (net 1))
 (segment (start 155.2 90.5) (end 135.1 90.5) (width 0.254) (layer B.Cu) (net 1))
 (segment (start 112.5 89) (end 117 89) (width 0.254) (layer B.Cu) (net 8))
 (segment (start 117 89) (end 122.5 94.5) (width 0.254) (layer B.Cu) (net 8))
 (via (at 130 94.5) (size 0.6) (drill 0.4) (layers F.Cu B.Cu) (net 8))
 (segment (start 130 88) (end 130 94.5) (width 0.254) (layer F.Cu) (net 8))
 (segment (start 122.5 94.5) (end 130 94.5) (width 0.254) (layer B.Cu) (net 8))
 (via (at 150 94.5) (size 0.6) (drill 0.4) (layers F.Cu B.Cu) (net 8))
 (segment (start 150 87.5) (end 150 94.5) (width 0.254) (layer F.Cu) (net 8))
 (segment (start 150 94.5) (end 130 94.5) (width 0.254) (layer B.Cu) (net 8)))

